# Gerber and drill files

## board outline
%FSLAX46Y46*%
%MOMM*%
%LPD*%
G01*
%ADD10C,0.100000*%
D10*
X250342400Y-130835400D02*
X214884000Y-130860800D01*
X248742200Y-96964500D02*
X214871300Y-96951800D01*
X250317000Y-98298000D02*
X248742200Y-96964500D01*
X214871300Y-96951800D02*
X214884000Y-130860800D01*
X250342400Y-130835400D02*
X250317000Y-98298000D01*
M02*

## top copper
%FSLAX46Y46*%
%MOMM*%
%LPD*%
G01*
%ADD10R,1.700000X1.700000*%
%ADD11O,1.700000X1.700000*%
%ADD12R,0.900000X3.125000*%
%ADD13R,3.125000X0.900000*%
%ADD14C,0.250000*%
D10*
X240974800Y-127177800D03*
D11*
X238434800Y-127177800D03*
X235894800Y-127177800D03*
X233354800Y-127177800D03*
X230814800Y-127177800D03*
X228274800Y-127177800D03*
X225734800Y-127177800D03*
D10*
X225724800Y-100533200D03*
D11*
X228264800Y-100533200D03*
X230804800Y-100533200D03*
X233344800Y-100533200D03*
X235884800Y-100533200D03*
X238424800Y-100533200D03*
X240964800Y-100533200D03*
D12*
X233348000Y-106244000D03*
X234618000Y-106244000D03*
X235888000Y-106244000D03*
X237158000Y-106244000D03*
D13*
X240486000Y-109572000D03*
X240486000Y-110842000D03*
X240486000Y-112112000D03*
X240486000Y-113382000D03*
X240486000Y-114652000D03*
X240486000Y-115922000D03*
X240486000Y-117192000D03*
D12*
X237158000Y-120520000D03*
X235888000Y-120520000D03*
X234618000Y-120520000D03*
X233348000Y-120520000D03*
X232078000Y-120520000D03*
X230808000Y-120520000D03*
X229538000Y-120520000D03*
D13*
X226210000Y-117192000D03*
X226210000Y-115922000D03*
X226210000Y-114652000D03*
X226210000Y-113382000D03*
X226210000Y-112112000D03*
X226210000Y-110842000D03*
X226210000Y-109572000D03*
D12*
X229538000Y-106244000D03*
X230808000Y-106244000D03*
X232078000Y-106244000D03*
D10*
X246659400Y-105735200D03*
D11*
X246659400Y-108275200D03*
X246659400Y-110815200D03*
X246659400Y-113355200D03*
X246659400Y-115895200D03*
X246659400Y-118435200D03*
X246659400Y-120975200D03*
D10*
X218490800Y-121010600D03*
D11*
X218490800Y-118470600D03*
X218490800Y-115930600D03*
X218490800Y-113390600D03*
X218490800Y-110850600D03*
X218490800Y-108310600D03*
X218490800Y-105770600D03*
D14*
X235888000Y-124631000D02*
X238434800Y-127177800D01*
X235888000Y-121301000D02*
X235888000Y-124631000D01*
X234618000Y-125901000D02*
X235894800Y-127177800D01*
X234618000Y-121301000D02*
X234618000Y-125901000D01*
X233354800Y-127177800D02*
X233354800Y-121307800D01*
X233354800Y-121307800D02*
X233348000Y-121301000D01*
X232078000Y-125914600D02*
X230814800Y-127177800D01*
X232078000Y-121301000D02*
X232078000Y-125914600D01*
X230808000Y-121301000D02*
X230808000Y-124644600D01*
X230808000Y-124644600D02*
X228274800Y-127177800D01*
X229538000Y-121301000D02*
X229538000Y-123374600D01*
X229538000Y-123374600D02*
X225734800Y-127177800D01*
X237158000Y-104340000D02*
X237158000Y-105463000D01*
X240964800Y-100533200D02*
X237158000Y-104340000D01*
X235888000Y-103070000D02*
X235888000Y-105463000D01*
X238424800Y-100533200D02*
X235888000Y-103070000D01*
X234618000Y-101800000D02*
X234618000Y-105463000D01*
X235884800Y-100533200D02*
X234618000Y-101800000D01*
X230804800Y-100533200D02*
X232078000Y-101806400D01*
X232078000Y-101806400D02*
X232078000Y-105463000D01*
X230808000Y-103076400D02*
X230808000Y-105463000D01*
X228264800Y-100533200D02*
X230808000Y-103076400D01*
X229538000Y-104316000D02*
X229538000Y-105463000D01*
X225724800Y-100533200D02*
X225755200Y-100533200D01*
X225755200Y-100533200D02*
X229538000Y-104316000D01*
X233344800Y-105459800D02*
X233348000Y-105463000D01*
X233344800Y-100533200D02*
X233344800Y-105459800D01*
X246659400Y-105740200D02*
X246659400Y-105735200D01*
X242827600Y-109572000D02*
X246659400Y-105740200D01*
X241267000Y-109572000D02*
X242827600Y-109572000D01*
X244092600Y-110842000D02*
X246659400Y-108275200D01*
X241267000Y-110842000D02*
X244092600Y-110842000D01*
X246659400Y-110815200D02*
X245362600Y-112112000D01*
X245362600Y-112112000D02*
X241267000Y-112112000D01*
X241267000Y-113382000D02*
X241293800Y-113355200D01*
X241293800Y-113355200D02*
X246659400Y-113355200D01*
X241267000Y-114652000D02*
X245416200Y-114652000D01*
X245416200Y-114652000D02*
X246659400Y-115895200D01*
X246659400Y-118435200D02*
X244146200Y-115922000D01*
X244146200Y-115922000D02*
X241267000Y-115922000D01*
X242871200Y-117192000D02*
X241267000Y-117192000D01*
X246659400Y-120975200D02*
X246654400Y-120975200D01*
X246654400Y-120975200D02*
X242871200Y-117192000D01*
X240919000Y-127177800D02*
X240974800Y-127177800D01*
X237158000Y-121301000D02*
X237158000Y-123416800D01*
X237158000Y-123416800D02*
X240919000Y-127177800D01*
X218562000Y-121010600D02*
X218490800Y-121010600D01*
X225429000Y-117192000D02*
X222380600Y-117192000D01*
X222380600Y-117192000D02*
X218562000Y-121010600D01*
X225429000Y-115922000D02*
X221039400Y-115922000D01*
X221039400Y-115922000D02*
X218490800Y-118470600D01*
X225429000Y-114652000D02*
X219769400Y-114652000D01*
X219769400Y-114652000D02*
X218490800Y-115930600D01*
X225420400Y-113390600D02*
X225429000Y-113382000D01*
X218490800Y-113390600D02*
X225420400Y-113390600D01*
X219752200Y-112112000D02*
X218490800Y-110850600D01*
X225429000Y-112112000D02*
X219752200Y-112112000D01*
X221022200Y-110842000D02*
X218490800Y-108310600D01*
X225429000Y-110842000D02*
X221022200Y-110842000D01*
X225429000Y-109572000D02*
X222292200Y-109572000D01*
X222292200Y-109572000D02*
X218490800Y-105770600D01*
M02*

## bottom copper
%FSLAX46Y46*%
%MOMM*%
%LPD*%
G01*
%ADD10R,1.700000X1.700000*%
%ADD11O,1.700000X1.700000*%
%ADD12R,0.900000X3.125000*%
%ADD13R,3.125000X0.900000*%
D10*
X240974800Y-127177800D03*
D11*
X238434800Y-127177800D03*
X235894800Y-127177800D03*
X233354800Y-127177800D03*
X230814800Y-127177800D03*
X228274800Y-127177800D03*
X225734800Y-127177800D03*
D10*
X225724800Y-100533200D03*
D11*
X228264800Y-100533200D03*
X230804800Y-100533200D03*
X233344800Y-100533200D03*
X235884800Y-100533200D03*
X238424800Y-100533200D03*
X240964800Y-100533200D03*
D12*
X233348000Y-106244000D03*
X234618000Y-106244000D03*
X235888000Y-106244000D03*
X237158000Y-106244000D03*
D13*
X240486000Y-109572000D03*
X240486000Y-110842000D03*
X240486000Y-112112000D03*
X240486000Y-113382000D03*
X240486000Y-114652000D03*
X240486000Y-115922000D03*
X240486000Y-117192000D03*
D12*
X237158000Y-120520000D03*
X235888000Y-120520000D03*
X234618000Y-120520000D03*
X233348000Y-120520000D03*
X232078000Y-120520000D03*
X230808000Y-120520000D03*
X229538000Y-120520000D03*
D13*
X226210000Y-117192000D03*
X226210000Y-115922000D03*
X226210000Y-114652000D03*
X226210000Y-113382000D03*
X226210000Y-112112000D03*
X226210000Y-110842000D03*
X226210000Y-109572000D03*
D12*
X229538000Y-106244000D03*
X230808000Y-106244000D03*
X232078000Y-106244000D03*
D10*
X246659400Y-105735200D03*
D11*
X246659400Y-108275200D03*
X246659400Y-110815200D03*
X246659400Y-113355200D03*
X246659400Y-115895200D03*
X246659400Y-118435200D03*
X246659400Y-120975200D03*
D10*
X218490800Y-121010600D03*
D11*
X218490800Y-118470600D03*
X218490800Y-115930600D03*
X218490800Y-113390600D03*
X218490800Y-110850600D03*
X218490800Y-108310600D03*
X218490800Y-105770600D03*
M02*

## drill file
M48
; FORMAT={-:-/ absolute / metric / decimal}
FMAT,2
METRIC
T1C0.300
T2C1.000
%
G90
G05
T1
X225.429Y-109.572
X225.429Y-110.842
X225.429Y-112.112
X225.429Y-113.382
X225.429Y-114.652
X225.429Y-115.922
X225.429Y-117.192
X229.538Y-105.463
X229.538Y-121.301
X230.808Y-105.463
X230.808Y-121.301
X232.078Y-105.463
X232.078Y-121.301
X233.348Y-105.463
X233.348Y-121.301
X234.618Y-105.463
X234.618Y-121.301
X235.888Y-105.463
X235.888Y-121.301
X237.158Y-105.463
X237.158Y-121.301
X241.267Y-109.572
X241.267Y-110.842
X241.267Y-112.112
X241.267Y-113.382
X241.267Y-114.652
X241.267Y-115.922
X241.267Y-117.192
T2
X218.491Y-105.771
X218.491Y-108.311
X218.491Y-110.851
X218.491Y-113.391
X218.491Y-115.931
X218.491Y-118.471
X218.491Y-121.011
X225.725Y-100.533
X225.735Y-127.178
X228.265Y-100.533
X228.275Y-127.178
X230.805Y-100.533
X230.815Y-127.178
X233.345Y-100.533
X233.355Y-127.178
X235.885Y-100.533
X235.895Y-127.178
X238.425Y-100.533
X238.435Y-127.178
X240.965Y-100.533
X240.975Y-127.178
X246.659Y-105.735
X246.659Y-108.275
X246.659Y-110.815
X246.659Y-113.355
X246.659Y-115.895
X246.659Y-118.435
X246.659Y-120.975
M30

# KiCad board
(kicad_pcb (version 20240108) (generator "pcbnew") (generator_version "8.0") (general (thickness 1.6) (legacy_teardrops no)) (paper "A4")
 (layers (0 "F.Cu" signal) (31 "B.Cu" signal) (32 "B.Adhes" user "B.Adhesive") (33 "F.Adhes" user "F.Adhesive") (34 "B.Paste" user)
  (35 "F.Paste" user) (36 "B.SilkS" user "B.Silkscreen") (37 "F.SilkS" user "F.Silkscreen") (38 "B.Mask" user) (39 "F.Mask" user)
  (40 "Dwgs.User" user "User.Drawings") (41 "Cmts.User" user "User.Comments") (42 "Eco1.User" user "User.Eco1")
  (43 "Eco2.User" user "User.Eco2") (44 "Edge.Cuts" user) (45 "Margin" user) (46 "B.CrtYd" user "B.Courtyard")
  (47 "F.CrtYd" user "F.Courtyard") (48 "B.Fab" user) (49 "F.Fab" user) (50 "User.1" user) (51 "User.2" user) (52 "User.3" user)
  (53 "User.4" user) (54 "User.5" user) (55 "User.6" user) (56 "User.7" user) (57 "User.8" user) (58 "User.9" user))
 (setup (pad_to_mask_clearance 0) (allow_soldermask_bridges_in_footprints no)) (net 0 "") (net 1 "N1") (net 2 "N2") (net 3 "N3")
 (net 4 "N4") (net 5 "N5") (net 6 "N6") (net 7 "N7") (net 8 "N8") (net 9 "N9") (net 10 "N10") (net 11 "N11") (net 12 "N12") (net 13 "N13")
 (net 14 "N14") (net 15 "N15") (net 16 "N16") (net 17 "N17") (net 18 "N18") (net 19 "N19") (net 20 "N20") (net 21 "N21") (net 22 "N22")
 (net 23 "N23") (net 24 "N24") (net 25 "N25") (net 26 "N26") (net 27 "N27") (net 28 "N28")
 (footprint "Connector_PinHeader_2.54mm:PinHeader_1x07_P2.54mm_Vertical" (layer "F.Cu") (at 240.9748 127.1778 -90)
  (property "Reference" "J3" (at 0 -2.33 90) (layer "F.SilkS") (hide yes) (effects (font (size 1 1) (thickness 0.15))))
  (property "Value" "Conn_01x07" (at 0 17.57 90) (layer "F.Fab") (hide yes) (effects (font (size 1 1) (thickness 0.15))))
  (pad "1" thru_hole rect (at 0 0 270) (size 1.7 1.7) (drill 1) (layers "*.Cu" "*.Mask") (remove_unused_layers no) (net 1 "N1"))
  (pad "2" thru_hole oval (at 0 2.54 270) (size 1.7 1.7) (drill 1) (layers "*.Cu" "*.Mask") (remove_unused_layers no) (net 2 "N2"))
  (pad "3" thru_hole oval (at 0 5.08 270) (size 1.7 1.7) (drill 1) (layers "*.Cu" "*.Mask") (remove_unused_layers no) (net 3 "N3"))
  (pad "4" thru_hole oval (at 0 7.62 270) (size 1.7 1.7) (drill 1) (layers "*.Cu" "*.Mask") (remove_unused_layers no) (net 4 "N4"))
  (pad "5" thru_hole oval (at 0 10.16 270) (size 1.7 1.7) (drill 1) (layers "*.Cu" "*.Mask") (remove_unused_layers no) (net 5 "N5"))
  (pad "6" thru_hole oval (at 0 12.7 270) (size 1.7 1.7) (drill 1) (layers "*.Cu" "*.Mask") (remove_unused_layers no) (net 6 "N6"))
  (pad "7" thru_hole oval (at 0 15.24 270) (size 1.7 1.7) (drill 1) (layers "*.Cu" "*.Mask") (remove_unused_layers no) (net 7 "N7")))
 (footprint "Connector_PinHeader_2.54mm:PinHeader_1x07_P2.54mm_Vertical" (layer "F.Cu") (at 225.7248 100.5332 90)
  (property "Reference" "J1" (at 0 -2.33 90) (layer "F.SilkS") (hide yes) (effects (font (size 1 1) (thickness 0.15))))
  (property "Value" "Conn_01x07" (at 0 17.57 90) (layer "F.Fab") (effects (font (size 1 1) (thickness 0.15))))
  (pad "1" thru_hole rect (at 0 0 90) (size 1.7 1.7) (drill 1) (layers "*.Cu" "*.Mask") (remove_unused_layers no) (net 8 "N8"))
  (pad "2" thru_hole oval (at 0 2.54 90) (size 1.7 1.7) (drill 1) (layers "*.Cu" "*.Mask") (remove_unused_layers no) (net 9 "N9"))
  (pad "3" thru_hole oval (at 0 5.08 90) (size 1.7 1.7) (drill 1) (layers "*.Cu" "*.Mask") (remove_unused_layers no) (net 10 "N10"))
  (pad "4" thru_hole oval (at 0 7.62 90) (size 1.7 1.7) (drill 1) (layers "*.Cu" "*.Mask") (remove_unused_layers no) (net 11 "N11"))
  (pad "5" thru_hole oval (at 0 10.16 90) (size 1.7 1.7) (drill 1) (layers "*.Cu" "*.Mask") (remove_unused_layers no) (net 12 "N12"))
  (pad "6" thru_hole oval (at 0 12.7 90) (size 1.7 1.7) (drill 1) (layers "*.Cu" "*.Mask") (remove_unused_layers no) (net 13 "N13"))
  (pad "7" thru_hole oval (at 0 15.24 90) (size 1.7 1.7) (drill 1) (layers "*.Cu" "*.Mask") (remove_unused_layers no) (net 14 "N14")))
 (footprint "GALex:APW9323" (layer "F.Cu") (at 233.348 113.382)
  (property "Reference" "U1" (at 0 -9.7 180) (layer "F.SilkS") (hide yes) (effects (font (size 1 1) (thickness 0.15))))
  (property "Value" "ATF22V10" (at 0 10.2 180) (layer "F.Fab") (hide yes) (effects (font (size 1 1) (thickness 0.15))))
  (pad "1" thru_hole rect (at 0 -7.919) (size 0.9 3.125) (drill 0.3 (offset 0 0.781)) (layers "*.Cu" "*.Mask") (remove_unused_layers no)
   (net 11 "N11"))
  (pad "2" thru_hole rect (at 1.27 -7.919) (size 0.9 3.125) (drill 0.3 (offset 0 0.781)) (layers "*.Cu" "*.Mask") (remove_unused_layers no)
   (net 12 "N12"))
  (pad "3" thru_hole rect (at 2.54 -7.919) (size 0.9 3.125) (drill 0.3 (offset 0 0.781)) (layers "*.Cu" "*.Mask") (remove_unused_layers no)
   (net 13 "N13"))
  (pad "4" thru_hole rect (at 3.81 -7.919) (size 0.9 3.125) (drill 0.3 (offset 0 0.781)) (layers "*.Cu" "*.Mask") (remove_unused_layers no)
   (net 14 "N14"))
  (pad "5" thru_hole rect (at 7.919 -3.81) (size 3.125 0.9) (drill 0.3 (offset -0.781 0)) (layers "*.Cu" "*.Mask") (remove_unused_layers no)
   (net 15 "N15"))
  (pad "6" thru_hole rect (at 7.919 -2.54) (size 3.125 0.9) (drill 0.3 (offset -0.781 0)) (layers "*.Cu" "*.Mask") (remove_unused_layers no)
   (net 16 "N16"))
  (pad "7" thru_hole rect (at 7.919 -1.27) (size 3.125 0.9) (drill 0.3 (offset -0.781 0)) (layers "*.Cu" "*.Mask") (remove_unused_layers no)
   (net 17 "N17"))
  (pad "8" thru_hole rect (at 7.919 0) (size 3.125 0.9) (drill 0.3 (offset -0.781 0)) (layers "*.Cu" "*.Mask") (remove_unused_layers no)
   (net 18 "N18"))
  (pad "9" thru_hole rect (at 7.919 1.27) (size 3.125 0.9) (drill 0.3 (offset -0.781 0)) (layers "*.Cu" "*.Mask") (remove_unused_layers no)
   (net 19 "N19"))
  (pad "10" thru_hole rect (at 7.919 2.54) (size 3.125 0.9) (drill 0.3 (offset -0.781 0)) (layers "*.Cu" "*.Mask") (remove_unused_layers no)
   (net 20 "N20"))
  (pad "11" thru_hole rect (at 7.919 3.81) (size 3.125 0.9) (drill 0.3 (offset -0.781 0)) (layers "*.Cu" "*.Mask") (remove_unused_layers no)
   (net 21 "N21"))
  (pad "12" thru_hole rect (at 3.81 7.919) (size 0.9 3.125) (drill 0.3 (offset 0 -0.781)) (layers "*.Cu" "*.Mask") (remove_unused_layers no)
   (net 1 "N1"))
  (pad "13" thru_hole rect (at 2.54 7.919) (size 0.9 3.125) (drill 0.3 (offset 0 -0.781)) (layers "*.Cu" "*.Mask") (remove_unused_layers no)
   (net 2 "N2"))
  (pad "14" thru_hole rect (at 1.27 7.919) (size 0.9 3.125) (drill 0.3 (offset 0 -0.781)) (layers "*.Cu" "*.Mask") (remove_unused_layers no)
   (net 3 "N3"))
  (pad "15" thru_hole rect (at 0 7.919) (size 0.9 3.125) (drill 0.3 (offset 0 -0.781)) (layers "*.Cu" "*.Mask") (remove_unused_layers no)
   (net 4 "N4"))
  (pad "16" thru_hole rect (at -1.27 7.919) (size 0.9 3.125) (drill 0.3 (offset 0 -0.781)) (layers "*.Cu" "*.Mask")
   (remove_unused_layers no) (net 5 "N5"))
  (pad "17" thru_hole rect (at -2.54 7.919) (size 0.9 3.125) (drill 0.3 (offset 0 -0.781)) (layers "*.Cu" "*.Mask")
   (remove_unused_layers no) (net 6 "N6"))
  (pad "18" thru_hole rect (at -3.81 7.919) (size 0.9 3.125) (drill 0.3 (offset 0 -0.781)) (layers "*.Cu" "*.Mask")
   (remove_unused_layers no) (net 7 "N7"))
  (pad "19" thru_hole rect (at -7.919 3.81) (size 3.125 0.9) (drill 0.3 (offset 0.781 0)) (layers "*.Cu" "*.Mask") (remove_unused_layers no)
   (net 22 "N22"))
  (pad "20" thru_hole rect (at -7.919 2.54) (size 3.125 0.9) (drill 0.3 (offset 0.781 0)) (layers "*.Cu" "*.Mask") (remove_unused_layers no)
   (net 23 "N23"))
  (pad "21" thru_hole rect (at -7.919 1.27) (size 3.125 0.9) (drill 0.3 (offset 0.781 0)) (layers "*.Cu" "*.Mask") (remove_unused_layers no)
   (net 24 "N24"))
  (pad "22" thru_hole rect (at -7.919 0) (size 3.125 0.9) (drill 0.3 (offset 0.781 0)) (layers "*.Cu" "*.Mask") (remove_unused_layers no)
   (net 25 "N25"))
  (pad "23" thru_hole rect (at -7.919 -1.27) (size 3.125 0.9) (drill 0.3 (offset 0.781 0)) (layers "*.Cu" "*.Mask")
   (remove_unused_layers no) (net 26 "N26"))
  (pad "24" thru_hole rect (at -7.919 -2.54) (size 3.125 0.9) (drill 0.3 (offset 0.781 0)) (layers "*.Cu" "*.Mask")
   (remove_unused_layers no) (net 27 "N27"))
  (pad "25" thru_hole rect (at -7.919 -3.81) (size 3.125 0.9) (drill 0.3 (offset 0.781 0)) (layers "*.Cu" "*.Mask")
   (remove_unused_layers no) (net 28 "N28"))
  (pad "26" thru_hole rect (at -3.81 -7.919) (size 0.9 3.125) (drill 0.3 (offset 0 0.781)) (layers "*.Cu" "*.Mask")
   (remove_unused_layers no) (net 8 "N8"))
  (pad "27" thru_hole rect (at -2.54 -7.919) (size 0.9 3.125) (drill 0.3 (offset 0 0.781)) (layers "*.Cu" "*.Mask")
   (remove_unused_layers no) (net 9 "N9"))
  (pad "28" thru_hole rect (at -1.27 -7.919) (size 0.9 3.125) (drill 0.3 (offset 0 0.781)) (layers "*.Cu" "*.Mask")
   (remove_unused_layers no) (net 10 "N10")))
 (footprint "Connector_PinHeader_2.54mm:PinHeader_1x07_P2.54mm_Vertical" (layer "F.Cu") (at 246.6594 105.7352)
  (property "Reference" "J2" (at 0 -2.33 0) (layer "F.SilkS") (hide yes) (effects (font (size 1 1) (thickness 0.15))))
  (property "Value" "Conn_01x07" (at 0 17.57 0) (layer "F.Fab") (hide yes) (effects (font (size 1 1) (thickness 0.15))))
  (pad "1" thru_hole rect (at 0 0) (size 1.7 1.7) (drill 1) (layers "*.Cu" "*.Mask") (remove_unused_layers no) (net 15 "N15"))
  (pad "2" thru_hole oval (at 0 2.54) (size 1.7 1.7) (drill 1) (layers "*.Cu" "*.Mask") (remove_unused_layers no) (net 16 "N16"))
  (pad "3" thru_hole oval (at 0 5.08) (size 1.7 1.7) (drill 1) (layers "*.Cu" "*.Mask") (remove_unused_layers no) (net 17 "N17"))
  (pad "4" thru_hole oval (at 0 7.62) (size 1.7 1.7) (drill 1) (layers "*.Cu" "*.Mask") (remove_unused_layers no) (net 18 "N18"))
  (pad "5" thru_hole oval (at 0 10.16) (size 1.7 1.7) (drill 1) (layers "*.Cu" "*.Mask") (remove_unused_layers no) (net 19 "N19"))
  (pad "6" thru_hole oval (at 0 12.7) (size 1.7 1.7) (drill 1) (layers "*.Cu" "*.Mask") (remove_unused_layers no) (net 20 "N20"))
  (pad "7" thru_hole oval (at 0 15.24) (size 1.7 1.7) (drill 1) (layers "*.Cu" "*.Mask") (remove_unused_layers no) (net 21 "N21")))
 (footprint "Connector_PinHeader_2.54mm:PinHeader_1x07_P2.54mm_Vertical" (layer "F.Cu") (at 218.4908 121.0106 180)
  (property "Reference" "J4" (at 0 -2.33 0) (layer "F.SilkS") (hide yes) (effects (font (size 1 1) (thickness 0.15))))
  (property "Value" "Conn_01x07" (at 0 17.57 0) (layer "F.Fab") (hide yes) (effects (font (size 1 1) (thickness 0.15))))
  (pad "1" thru_hole rect (at 0 0 180) (size 1.7 1.7) (drill 1) (layers "*.Cu" "*.Mask") (remove_unused_layers no) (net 22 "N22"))
  (pad "2" thru_hole oval (at 0 2.54 180) (size 1.7 1.7) (drill 1) (layers "*.Cu" "*.Mask") (remove_unused_layers no) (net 23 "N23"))
  (pad "3" thru_hole oval (at 0 5.08 180) (size 1.7 1.7) (drill 1) (layers "*.Cu" "*.Mask") (remove_unused_layers no) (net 24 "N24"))
  (pad "4" thru_hole oval (at 0 7.62 180) (size 1.7 1.7) (drill 1) (layers "*.Cu" "*.Mask") (remove_unused_layers no) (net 25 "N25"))
  (pad "5" thru_hole oval (at 0 10.16 180) (size 1.7 1.7) (drill 1) (layers "*.Cu" "*.Mask") (remove_unused_layers no) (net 26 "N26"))
  (pad "6" thru_hole oval (at 0 12.7 180) (size 1.7 1.7) (drill 1) (layers "*.Cu" "*.Mask") (remove_unused_layers no) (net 27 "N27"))
  (pad "7" thru_hole oval (at 0 15.24 180) (size 1.7 1.7) (drill 1) (layers "*.Cu" "*.Mask") (remove_unused_layers no) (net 28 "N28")))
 (gr_line (start 250.3424 130.8354) (end 214.884 130.8608) (stroke (width 0.1) (type solid)) (layer "Edge.Cuts"))
 (gr_line (start 248.7422 96.9645) (end 214.8713 96.9518) (stroke (width 0.1) (type solid)) (layer "Edge.Cuts"))
 (gr_line (start 250.317 98.298) (end 248.7422 96.9645) (stroke (width 0.1) (type solid)) (layer "Edge.Cuts"))
 (gr_line (start 214.8713 96.9518) (end 214.884 130.8608) (stroke (width 0.1) (type solid)) (layer "Edge.Cuts"))
 (gr_line (start 250.3424 130.8354) (end 250.317 98.298) (stroke (width 0.1) (type solid)) (layer "Edge.Cuts"))
 (segment (start 235.888 124.631) (end 238.4348 127.1778) (width 0.25) (layer "F.Cu") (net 2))
 (segment (start 235.888 121.301) (end 235.888 124.631) (width 0.25) (layer "F.Cu") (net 2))
 (segment (start 234.618 125.901) (end 235.8948 127.1778) (width 0.25) (layer "F.Cu") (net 3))
 (segment (start 234.618 121.301) (end 234.618 125.901) (width 0.25) (layer "F.Cu") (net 3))
 (segment (start 233.3548 127.1778) (end 233.3548 121.3078) (width 0.25) (layer "F.Cu") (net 4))
 (segment (start 233.3548 121.3078) (end 233.348 121.301) (width 0.25) (layer "F.Cu") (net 4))
 (segment (start 232.078 125.9146) (end 230.8148 127.1778) (width 0.25) (layer "F.Cu") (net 5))
 (segment (start 232.078 121.301) (end 232.078 125.9146) (width 0.25) (layer "F.Cu") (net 5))
 (segment (start 230.808 121.301) (end 230.808 124.6446) (width 0.25) (layer "F.Cu") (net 6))
 (segment (start 230.808 124.6446) (end 228.2748 127.1778) (width 0.25) (layer "F.Cu") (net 6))
 (segment (start 229.538 121.301) (end 229.538 123.3746) (width 0.25) (layer "F.Cu") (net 7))
 (segment (start 229.538 123.3746) (end 225.7348 127.1778) (width 0.25) (layer "F.Cu") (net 7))
 (segment (start 237.158 104.34) (end 237.158 105.463) (width 0.25) (layer "F.Cu") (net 14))
 (segment (start 240.9648 100.5332) (end 237.158 104.34) (width 0.25) (layer "F.Cu") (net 14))
 (segment (start 235.888 103.07) (end 235.888 105.463) (width 0.25) (layer "F.Cu") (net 13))
 (segment (start 238.4248 100.5332) (end 235.888 103.07) (width 0.25) (layer "F.Cu") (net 13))
 (segment (start 234.618 101.8) (end 234.618 105.463) (width 0.25) (layer "F.Cu") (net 12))
 (segment (start 235.8848 100.5332) (end 234.618 101.8) (width 0.25) (layer "F.Cu") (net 12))
 (segment (start 230.8048 100.5332) (end 232.078 101.8064) (width 0.25) (layer "F.Cu") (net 10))
 (segment (start 232.078 101.8064) (end 232.078 105.463) (width 0.25) (layer "F.Cu") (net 10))
 (segment (start 230.808 103.0764) (end 230.808 105.463) (width 0.25) (layer "F.Cu") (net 9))
 (segment (start 228.2648 100.5332) (end 230.808 103.0764) (width 0.25) (layer "F.Cu") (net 9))
 (segment (start 229.538 104.316) (end 229.538 105.463) (width 0.25) (layer "F.Cu") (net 8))
 (segment (start 225.7248 100.5332) (end 225.7552 100.5332) (width 0.25) (layer "F.Cu") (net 8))
 (segment (start 225.7552 100.5332) (end 229.538 104.316) (width 0.25) (layer "F.Cu") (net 8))
 (segment (start 233.3448 105.4598) (end 233.348 105.463) (width 0.25) (layer "F.Cu") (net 11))
 (segment (start 233.3448 100.5332) (end 233.3448 105.4598) (width 0.25) (layer "F.Cu") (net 11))
 (segment (start 246.6594 105.7402) (end 246.6594 105.7352) (width 0.25) (layer "F.Cu") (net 15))
 (segment (start 242.8276 109.572) (end 246.6594 105.7402) (width 0.25) (layer "F.Cu") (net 15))
 (segment (start 241.267 109.572) (end 242.8276 109.572) (width 0.25) (layer "F.Cu") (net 15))
 (segment (start 244.0926 110.842) (end 246.6594 108.2752) (width 0.25) (layer "F.Cu") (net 16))
 (segment (start 241.267 110.842) (end 244.0926 110.842) (width 0.25) (layer "F.Cu") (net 16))
 (segment (start 246.6594 110.8152) (end 245.3626 112.112) (width 0.25) (layer "F.Cu") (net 17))
 (segment (start 245.3626 112.112) (end 241.267 112.112) (width 0.25) (layer "F.Cu") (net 17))
 (segment (start 241.267 113.382) (end 241.2938 113.3552) (width 0.25) (layer "F.Cu") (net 18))
 (segment (start 241.2938 113.3552) (end 246.6594 113.3552) (width 0.25) (layer "F.Cu") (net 18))
 (segment (start 241.267 114.652) (end 245.4162 114.652) (width 0.25) (layer "F.Cu") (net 19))
 (segment (start 245.4162 114.652) (end 246.6594 115.8952) (width 0.25) (layer "F.Cu") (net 19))
 (segment (start 246.6594 118.4352) (end 244.1462 115.922) (width 0.25) (layer "F.Cu") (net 20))
 (segment (start 244.1462 115.922) (end 241.267 115.922) (width 0.25) (layer "F.Cu") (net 20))
 (segment (start 242.8712 117.192) (end 241.267 117.192) (width 0.25) (layer "F.Cu") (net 21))
 (segment (start 246.6594 120.9752) (end 246.6544 120.9752) (width 0.25) (layer "F.Cu") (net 21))
 (segment (start 246.6544 120.9752) (end 242.8712 117.192) (width 0.25) (layer "F.Cu") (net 21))
 (segment (start 240.919 127.1778) (end 240.9748 127.1778) (width 0.25) (layer "F.Cu") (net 1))
 (segment (start 237.158 121.301) (end 237.158 123.4168) (width 0.25) (layer "F.Cu") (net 1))
 (segment (start 237.158 123.4168) (end 240.919 127.1778) (width 0.25) (layer "F.Cu") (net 1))
 (segment (start 218.562 121.0106) (end 218.4908 121.0106) (width 0.25) (layer "F.Cu") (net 22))
 (segment (start 225.429 117.192) (end 222.3806 117.192) (width 0.25) (layer "F.Cu") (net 22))
 (segment (start 222.3806 117.192) (end 218.562 121.0106) (width 0.25) (layer "F.Cu") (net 22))
 (segment (start 225.429 115.922) (end 221.0394 115.922) (width 0.25) (layer "F.Cu") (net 23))
 (segment (start 221.0394 115.922) (end 218.4908 118.4706) (width 0.25) (layer "F.Cu") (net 23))
 (segment (start 225.429 114.652) (end 219.7694 114.652) (width 0.25) (layer "F.Cu") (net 24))
 (segment (start 219.7694 114.652) (end 218.4908 115.9306) (width 0.25) (layer "F.Cu") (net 24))
 (segment (start 225.4204 113.3906) (end 225.429 113.382) (width 0.25) (layer "F.Cu") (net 25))
 (segment (start 218.4908 113.3906) (end 225.4204 113.3906) (width 0.25) (layer "F.Cu") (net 25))
 (segment (start 219.7522 112.112) (end 218.4908 110.8506) (width 0.25) (layer "F.Cu") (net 26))
 (segment (start 225.429 112.112) (end 219.7522 112.112) (width 0.25) (layer "F.Cu") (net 26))
 (segment (start 221.0222 110.842) (end 218.4908 108.3106) (width 0.25) (layer "F.Cu") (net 27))
 (segment (start 225.429 110.842) (end 221.0222 110.842) (width 0.25) (layer "F.Cu") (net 27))
 (segment (start 225.429 109.572) (end 222.2922 109.572) (width 0.25) (layer "F.Cu") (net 28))
 (segment (start 222.2922 109.572) (end 218.4908 105.7706) (width 0.25) (layer "F.Cu") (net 28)))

